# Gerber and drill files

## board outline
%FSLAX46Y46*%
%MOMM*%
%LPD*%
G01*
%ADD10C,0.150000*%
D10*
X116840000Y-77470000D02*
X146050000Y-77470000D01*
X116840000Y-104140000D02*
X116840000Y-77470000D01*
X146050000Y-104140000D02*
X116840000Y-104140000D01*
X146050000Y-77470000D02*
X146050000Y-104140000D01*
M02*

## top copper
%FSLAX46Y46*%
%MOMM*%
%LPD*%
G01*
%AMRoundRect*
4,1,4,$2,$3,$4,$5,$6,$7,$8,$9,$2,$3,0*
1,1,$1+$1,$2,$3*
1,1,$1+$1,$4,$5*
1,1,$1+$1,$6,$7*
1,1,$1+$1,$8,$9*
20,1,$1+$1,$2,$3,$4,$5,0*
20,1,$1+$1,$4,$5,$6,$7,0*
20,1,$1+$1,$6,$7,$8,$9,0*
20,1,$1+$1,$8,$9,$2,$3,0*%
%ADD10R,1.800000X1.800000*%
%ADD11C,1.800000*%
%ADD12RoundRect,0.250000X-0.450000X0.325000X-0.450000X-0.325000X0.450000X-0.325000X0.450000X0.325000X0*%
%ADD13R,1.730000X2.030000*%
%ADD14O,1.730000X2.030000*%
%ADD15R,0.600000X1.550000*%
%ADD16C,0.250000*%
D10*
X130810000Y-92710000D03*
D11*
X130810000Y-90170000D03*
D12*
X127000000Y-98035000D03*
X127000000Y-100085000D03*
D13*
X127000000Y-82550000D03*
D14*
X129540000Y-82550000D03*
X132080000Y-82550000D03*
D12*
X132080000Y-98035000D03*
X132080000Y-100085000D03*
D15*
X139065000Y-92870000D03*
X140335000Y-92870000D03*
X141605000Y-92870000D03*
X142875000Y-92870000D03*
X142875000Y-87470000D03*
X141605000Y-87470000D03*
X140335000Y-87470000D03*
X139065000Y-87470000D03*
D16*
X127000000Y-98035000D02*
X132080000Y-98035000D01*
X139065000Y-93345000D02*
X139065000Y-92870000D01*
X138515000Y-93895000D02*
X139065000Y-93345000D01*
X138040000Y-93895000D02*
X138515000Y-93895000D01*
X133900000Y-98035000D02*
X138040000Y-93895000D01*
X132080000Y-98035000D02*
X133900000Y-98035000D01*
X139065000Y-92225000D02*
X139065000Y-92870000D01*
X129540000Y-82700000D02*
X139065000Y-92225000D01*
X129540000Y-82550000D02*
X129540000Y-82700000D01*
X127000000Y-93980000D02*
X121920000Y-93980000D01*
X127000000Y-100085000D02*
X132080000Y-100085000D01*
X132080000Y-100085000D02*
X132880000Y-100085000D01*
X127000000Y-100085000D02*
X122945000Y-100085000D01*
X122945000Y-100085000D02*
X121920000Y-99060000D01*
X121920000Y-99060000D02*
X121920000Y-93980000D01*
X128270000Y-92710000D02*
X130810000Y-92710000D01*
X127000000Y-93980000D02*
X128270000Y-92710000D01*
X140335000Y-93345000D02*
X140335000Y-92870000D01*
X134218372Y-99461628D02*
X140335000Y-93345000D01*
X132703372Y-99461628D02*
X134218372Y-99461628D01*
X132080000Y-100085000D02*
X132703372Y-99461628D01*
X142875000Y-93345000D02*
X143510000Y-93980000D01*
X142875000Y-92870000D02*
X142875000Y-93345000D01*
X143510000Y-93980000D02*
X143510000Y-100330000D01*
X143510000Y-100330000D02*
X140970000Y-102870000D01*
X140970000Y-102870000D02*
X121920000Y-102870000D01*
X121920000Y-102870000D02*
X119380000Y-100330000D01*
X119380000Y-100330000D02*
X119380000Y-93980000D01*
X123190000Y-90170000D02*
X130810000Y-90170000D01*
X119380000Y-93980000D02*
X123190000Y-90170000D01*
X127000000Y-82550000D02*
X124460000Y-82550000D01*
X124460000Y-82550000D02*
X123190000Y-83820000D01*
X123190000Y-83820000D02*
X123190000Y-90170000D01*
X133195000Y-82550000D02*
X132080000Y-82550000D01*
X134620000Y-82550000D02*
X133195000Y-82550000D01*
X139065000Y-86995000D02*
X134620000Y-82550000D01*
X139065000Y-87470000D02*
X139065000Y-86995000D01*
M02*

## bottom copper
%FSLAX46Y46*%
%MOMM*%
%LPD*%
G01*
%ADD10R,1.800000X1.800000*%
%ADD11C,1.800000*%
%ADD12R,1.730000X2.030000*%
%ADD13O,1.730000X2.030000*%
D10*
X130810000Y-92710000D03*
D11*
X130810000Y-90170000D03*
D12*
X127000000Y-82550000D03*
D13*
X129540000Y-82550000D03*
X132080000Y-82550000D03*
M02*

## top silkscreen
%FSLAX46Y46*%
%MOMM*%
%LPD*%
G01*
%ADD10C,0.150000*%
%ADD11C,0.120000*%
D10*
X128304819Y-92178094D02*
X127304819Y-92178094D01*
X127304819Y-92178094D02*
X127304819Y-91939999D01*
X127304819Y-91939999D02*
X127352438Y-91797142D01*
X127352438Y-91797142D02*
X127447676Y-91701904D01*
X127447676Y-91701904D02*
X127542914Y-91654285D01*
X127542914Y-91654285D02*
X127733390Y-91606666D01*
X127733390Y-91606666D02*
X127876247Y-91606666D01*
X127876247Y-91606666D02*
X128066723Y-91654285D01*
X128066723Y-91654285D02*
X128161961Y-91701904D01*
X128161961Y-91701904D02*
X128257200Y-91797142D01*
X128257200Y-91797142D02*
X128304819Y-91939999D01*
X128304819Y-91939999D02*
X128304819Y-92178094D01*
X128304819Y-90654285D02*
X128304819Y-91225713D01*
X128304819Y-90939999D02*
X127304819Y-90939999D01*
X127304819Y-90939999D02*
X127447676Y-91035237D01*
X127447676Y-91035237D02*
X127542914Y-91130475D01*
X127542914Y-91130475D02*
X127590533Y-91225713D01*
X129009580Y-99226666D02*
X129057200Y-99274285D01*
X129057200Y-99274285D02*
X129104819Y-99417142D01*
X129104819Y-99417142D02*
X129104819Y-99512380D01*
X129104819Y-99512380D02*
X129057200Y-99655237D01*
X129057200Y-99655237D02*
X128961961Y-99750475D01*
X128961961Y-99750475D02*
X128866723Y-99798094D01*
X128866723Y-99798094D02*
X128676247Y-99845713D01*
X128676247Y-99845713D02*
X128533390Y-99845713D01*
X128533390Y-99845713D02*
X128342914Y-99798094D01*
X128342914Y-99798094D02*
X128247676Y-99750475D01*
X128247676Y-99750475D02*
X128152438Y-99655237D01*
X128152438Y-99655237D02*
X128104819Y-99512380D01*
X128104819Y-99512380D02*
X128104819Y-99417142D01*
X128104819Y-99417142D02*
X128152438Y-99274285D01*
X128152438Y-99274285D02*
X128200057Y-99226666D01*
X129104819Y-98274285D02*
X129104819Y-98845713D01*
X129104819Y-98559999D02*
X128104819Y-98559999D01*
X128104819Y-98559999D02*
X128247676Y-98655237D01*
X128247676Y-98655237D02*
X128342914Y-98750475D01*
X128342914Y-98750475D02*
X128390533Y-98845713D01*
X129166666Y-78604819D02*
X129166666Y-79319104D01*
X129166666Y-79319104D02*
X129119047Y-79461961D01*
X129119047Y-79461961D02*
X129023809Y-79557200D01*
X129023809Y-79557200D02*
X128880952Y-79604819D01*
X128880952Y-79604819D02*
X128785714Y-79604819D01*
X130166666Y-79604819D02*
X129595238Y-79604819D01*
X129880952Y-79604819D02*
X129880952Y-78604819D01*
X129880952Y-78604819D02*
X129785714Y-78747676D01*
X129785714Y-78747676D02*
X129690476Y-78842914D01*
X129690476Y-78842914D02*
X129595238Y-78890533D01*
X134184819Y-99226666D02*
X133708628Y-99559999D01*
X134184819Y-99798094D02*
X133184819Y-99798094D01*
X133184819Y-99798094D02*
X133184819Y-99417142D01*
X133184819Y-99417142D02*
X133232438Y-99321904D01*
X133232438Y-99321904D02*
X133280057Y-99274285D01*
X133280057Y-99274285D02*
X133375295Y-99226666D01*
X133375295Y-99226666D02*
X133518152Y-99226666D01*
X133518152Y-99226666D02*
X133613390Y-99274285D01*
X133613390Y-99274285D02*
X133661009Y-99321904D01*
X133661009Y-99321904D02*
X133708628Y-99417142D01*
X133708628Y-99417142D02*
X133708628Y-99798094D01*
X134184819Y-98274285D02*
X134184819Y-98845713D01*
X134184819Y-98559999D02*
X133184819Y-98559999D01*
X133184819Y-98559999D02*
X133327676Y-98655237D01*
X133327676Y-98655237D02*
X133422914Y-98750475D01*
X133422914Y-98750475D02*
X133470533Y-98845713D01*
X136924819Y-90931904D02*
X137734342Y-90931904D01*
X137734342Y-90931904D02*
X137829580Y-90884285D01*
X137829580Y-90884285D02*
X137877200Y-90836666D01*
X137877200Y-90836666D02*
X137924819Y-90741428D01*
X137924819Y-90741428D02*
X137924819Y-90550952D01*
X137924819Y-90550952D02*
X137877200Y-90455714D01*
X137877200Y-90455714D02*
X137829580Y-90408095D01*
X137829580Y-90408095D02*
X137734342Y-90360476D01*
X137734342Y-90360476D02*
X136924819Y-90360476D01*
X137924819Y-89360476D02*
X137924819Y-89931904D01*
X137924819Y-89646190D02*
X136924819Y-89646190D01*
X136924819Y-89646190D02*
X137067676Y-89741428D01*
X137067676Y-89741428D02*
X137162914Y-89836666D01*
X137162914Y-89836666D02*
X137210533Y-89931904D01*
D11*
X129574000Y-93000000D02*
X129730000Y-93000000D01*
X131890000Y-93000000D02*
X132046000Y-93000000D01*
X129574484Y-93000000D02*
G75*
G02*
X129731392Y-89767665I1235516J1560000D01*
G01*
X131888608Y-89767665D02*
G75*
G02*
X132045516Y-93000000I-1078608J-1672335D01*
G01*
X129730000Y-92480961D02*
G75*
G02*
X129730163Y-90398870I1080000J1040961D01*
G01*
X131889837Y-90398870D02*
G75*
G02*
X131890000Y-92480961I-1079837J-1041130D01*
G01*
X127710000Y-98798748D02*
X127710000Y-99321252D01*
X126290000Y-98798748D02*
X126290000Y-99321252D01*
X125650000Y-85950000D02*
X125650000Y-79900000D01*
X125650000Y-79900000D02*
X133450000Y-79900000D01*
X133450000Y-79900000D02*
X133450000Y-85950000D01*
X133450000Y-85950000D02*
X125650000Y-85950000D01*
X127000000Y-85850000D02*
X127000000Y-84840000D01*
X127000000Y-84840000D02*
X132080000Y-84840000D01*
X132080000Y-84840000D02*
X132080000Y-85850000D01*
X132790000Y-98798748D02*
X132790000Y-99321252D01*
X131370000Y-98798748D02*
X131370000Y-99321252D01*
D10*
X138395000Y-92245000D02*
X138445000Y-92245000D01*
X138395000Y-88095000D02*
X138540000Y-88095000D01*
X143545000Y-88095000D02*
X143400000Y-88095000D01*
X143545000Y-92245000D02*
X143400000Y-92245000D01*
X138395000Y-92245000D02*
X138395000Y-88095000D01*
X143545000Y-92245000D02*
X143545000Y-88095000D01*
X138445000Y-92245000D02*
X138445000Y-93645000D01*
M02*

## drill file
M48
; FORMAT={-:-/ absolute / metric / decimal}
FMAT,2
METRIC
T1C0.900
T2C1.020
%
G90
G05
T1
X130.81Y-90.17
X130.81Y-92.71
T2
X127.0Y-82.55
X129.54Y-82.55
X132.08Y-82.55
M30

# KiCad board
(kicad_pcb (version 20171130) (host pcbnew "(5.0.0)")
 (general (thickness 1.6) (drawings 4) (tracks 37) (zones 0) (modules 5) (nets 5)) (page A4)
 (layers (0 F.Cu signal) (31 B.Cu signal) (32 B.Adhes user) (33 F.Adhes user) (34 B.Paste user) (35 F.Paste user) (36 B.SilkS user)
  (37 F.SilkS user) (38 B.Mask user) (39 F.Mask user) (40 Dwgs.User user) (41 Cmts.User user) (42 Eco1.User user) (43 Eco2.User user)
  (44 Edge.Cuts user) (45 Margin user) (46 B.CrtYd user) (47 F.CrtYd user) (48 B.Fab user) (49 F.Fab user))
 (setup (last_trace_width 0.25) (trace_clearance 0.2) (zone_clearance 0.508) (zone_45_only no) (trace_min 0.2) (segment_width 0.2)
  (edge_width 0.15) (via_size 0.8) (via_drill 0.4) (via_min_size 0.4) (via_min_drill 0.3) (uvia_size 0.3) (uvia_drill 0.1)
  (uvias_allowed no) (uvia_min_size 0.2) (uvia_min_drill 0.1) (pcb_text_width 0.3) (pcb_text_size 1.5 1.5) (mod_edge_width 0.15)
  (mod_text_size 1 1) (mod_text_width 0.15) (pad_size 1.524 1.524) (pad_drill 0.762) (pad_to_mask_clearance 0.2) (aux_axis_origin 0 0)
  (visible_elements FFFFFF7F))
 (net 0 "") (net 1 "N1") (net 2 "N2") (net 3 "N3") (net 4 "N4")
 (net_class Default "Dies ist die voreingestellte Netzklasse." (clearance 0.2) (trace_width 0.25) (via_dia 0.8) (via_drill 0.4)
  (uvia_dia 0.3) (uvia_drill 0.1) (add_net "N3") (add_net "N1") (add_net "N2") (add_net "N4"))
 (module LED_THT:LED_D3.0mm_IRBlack (layer F.Cu) (at 130.81 92.71 90)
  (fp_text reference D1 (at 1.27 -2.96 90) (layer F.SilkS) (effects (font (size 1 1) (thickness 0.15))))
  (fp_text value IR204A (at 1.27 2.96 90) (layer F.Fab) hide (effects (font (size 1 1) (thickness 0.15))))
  (fp_line (start -0.29 -1.236) (end -0.29 -1.08) (layer F.SilkS) (width 0.12))
  (fp_line (start -0.29 1.08) (end -0.29 1.236) (layer F.SilkS) (width 0.12))
  (fp_arc (start 1.27 0) (end -0.29 -1.235516) (angle 108.8) (layer F.SilkS) (width 0.12))
  (fp_arc (start 1.27 0) (end -0.29 1.235516) (angle -108.8) (layer F.SilkS) (width 0.12))
  (fp_arc (start 1.27 0) (end 0.229039 -1.08) (angle 87.9) (layer F.SilkS) (width 0.12))
  (fp_arc (start 1.27 0) (end 0.229039 1.08) (angle -87.9) (layer F.SilkS) (width 0.12))
  (pad 1 thru_hole rect (at 0 0 90) (size 1.8 1.8) (drill 0.9) (layers *.Cu *.Mask) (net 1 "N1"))
  (pad 2 thru_hole circle (at 2.54 0 90) (size 1.8 1.8) (drill 0.9) (layers *.Cu *.Mask) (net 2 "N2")))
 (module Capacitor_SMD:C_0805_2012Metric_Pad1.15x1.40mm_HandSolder (layer F.Cu) (at 127 99.06 270)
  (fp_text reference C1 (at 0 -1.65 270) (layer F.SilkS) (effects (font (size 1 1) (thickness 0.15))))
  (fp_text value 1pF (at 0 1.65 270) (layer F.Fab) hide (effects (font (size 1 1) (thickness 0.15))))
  (fp_line (start -0.261252 -0.71) (end 0.261252 -0.71) (layer F.SilkS) (width 0.12))
  (fp_line (start -0.261252 0.71) (end 0.261252 0.71) (layer F.SilkS) (width 0.12))
  (pad 1 smd roundrect (at -1.025 0 270) (size 1.15 1.4) (layers F.Cu F.Paste F.Mask) (roundrect_rratio 0.217391) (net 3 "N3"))
  (pad 2 smd roundrect (at 1.025 0 270) (size 1.15 1.4) (layers F.Cu F.Paste F.Mask) (roundrect_rratio 0.217391) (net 1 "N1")))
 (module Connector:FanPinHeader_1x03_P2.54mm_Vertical (layer F.Cu) (at 127 82.55)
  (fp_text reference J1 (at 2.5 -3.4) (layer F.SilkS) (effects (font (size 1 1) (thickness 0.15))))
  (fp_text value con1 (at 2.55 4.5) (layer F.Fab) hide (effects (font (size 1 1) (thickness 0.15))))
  (fp_line (start -1.35 3.4) (end -1.35 -2.65) (layer F.SilkS) (width 0.12))
  (fp_line (start -1.35 -2.65) (end 6.45 -2.65) (layer F.SilkS) (width 0.12))
  (fp_line (start 6.45 -2.65) (end 6.45 3.4) (layer F.SilkS) (width 0.12))
  (fp_line (start 6.45 3.4) (end -1.35 3.4) (layer F.SilkS) (width 0.12))
  (fp_line (start 0 3.3) (end 0 2.29) (layer F.SilkS) (width 0.12))
  (fp_line (start 0 2.29) (end 5.08 2.29) (layer F.SilkS) (width 0.12))
  (fp_line (start 5.08 2.29) (end 5.08 3.3) (layer F.SilkS) (width 0.12))
  (pad 1 thru_hole rect (at 0 0 90) (size 2.03 1.73) (drill 1.02) (layers *.Cu *.Mask) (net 2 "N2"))
  (pad 2 thru_hole oval (at 2.54 0 90) (size 2.03 1.73) (drill 1.02) (layers *.Cu *.Mask) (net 3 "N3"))
  (pad 3 thru_hole oval (at 5.08 0 90) (size 2.03 1.73) (drill 1.02) (layers *.Cu *.Mask) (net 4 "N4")))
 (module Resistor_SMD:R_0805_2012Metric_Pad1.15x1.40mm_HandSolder (layer F.Cu) (at 132.08 99.06 270)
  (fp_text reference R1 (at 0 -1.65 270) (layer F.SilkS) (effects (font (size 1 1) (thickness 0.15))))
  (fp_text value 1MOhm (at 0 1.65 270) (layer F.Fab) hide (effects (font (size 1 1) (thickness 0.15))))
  (fp_line (start -0.261252 -0.71) (end 0.261252 -0.71) (layer F.SilkS) (width 0.12))
  (fp_line (start -0.261252 0.71) (end 0.261252 0.71) (layer F.SilkS) (width 0.12))
  (pad 1 smd roundrect (at -1.025 0 270) (size 1.15 1.4) (layers F.Cu F.Paste F.Mask) (roundrect_rratio 0.217391) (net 3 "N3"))
  (pad 2 smd roundrect (at 1.025 0 270) (size 1.15 1.4) (layers F.Cu F.Paste F.Mask) (roundrect_rratio 0.217391) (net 1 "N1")))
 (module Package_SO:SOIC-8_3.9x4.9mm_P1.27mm (layer F.Cu) (at 140.97 90.17 90)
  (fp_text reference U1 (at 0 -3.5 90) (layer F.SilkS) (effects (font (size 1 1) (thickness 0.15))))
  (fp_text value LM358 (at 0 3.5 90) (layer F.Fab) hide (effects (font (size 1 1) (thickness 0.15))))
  (fp_line (start -2.075 -2.575) (end -2.075 -2.525) (layer F.SilkS) (width 0.15))
  (fp_line (start 2.075 -2.575) (end 2.075 -2.43) (layer F.SilkS) (width 0.15))
  (fp_line (start 2.075 2.575) (end 2.075 2.43) (layer F.SilkS) (width 0.15))
  (fp_line (start -2.075 2.575) (end -2.075 2.43) (layer F.SilkS) (width 0.15))
  (fp_line (start -2.075 -2.575) (end 2.075 -2.575) (layer F.SilkS) (width 0.15))
  (fp_line (start -2.075 2.575) (end 2.075 2.575) (layer F.SilkS) (width 0.15))
  (fp_line (start -2.075 -2.525) (end -3.475 -2.525) (layer F.SilkS) (width 0.15))
  (pad 1 smd rect (at -2.7 -1.905 90) (size 1.55 0.6) (layers F.Cu F.Paste F.Mask) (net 3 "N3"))
  (pad 2 smd rect (at -2.7 -0.635 90) (size 1.55 0.6) (layers F.Cu F.Paste F.Mask) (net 1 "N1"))
  (pad 3 smd rect (at -2.7 0.635 90) (size 1.55 0.6) (layers F.Cu F.Paste F.Mask) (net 2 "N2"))
  (pad 4 smd rect (at -2.7 1.905 90) (size 1.55 0.6) (layers F.Cu F.Paste F.Mask) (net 2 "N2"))
  (pad 5 smd rect (at 2.7 1.905 90) (size 1.55 0.6) (layers F.Cu F.Paste F.Mask))
  (pad 6 smd rect (at 2.7 0.635 90) (size 1.55 0.6) (layers F.Cu F.Paste F.Mask))
  (pad 7 smd rect (at 2.7 -0.635 90) (size 1.55 0.6) (layers F.Cu F.Paste F.Mask))
  (pad 8 smd rect (at 2.7 -1.905 90) (size 1.55 0.6) (layers F.Cu F.Paste F.Mask) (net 4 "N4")))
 (gr_line (start 116.84 77.47) (end 146.05 77.47) (layer Edge.Cuts) (width 0.15))
 (gr_line (start 116.84 104.14) (end 116.84 77.47) (layer Edge.Cuts) (width 0.15))
 (gr_line (start 146.05 104.14) (end 116.84 104.14) (layer Edge.Cuts) (width 0.15))
 (gr_line (start 146.05 77.47) (end 146.05 104.14) (layer Edge.Cuts) (width 0.15))
 (segment (start 127 98.035) (end 132.08 98.035) (width 0.25) (layer F.Cu) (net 3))
 (segment (start 139.065 93.345) (end 139.065 92.87) (width 0.25) (layer F.Cu) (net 3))
 (segment (start 138.515 93.895) (end 139.065 93.345) (width 0.25) (layer F.Cu) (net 3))
 (segment (start 138.04 93.895) (end 138.515 93.895) (width 0.25) (layer F.Cu) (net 3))
 (segment (start 133.9 98.035) (end 138.04 93.895) (width 0.25) (layer F.Cu) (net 3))
 (segment (start 132.08 98.035) (end 133.9 98.035) (width 0.25) (layer F.Cu) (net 3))
 (segment (start 139.065 92.225) (end 139.065 92.87) (width 0.25) (layer F.Cu) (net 3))
 (segment (start 129.54 82.7) (end 139.065 92.225) (width 0.25) (layer F.Cu) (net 3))
 (segment (start 129.54 82.55) (end 129.54 82.7) (width 0.25) (layer F.Cu) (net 3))
 (segment (start 127 93.98) (end 121.92 93.98) (width 0.25) (layer F.Cu) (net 1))
 (segment (start 127 100.085) (end 132.08 100.085) (width 0.25) (layer F.Cu) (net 1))
 (segment (start 132.08 100.085) (end 132.88 100.085) (width 0.25) (layer F.Cu) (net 1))
 (segment (start 127 100.085) (end 122.945 100.085) (width 0.25) (layer F.Cu) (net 1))
 (segment (start 122.945 100.085) (end 121.92 99.06) (width 0.25) (layer F.Cu) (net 1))
 (segment (start 121.92 99.06) (end 121.92 93.98) (width 0.25) (layer F.Cu) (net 1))
 (segment (start 128.27 92.71) (end 130.81 92.71) (width 0.25) (layer F.Cu) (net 1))
 (segment (start 127 93.98) (end 128.27 92.71) (width 0.25) (layer F.Cu) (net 1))
 (segment (start 140.335 93.345) (end 140.335 92.87) (width 0.25) (layer F.Cu) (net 1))
 (segment (start 134.218372 99.461628) (end 140.335 93.345) (width 0.25) (layer F.Cu) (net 1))
 (segment (start 132.703372 99.461628) (end 134.218372 99.461628) (width 0.25) (layer F.Cu) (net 1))
 (segment (start 132.08 100.085) (end 132.703372 99.461628) (width 0.25) (layer F.Cu) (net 1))
 (segment (start 142.875 93.345) (end 143.51 93.98) (width 0.25) (layer F.Cu) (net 2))
 (segment (start 142.875 92.87) (end 142.875 93.345) (width 0.25) (layer F.Cu) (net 2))
 (segment (start 143.51 93.98) (end 143.51 100.33) (width 0.25) (layer F.Cu) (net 2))
 (segment (start 143.51 100.33) (end 140.97 102.87) (width 0.25) (layer F.Cu) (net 2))
 (segment (start 140.97 102.87) (end 121.92 102.87) (width 0.25) (layer F.Cu) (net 2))
 (segment (start 121.92 102.87) (end 119.38 100.33) (width 0.25) (layer F.Cu) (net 2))
 (segment (start 119.38 100.33) (end 119.38 93.98) (width 0.25) (layer F.Cu) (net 2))
 (segment (start 123.19 90.17) (end 130.81 90.17) (width 0.25) (layer F.Cu) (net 2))
 (segment (start 119.38 93.98) (end 123.19 90.17) (width 0.25) (layer F.Cu) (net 2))
 (segment (start 127 82.55) (end 124.46 82.55) (width 0.25) (layer F.Cu) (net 2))
 (segment (start 124.46 82.55) (end 123.19 83.82) (width 0.25) (layer F.Cu) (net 2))
 (segment (start 123.19 83.82) (end 123.19 90.17) (width 0.25) (layer F.Cu) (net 2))
 (segment (start 133.195 82.55) (end 132.08 82.55) (width 0.25) (layer F.Cu) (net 4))
 (segment (start 134.62 82.55) (end 133.195 82.55) (width 0.25) (layer F.Cu) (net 4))
 (segment (start 139.065 86.995) (end 134.62 82.55) (width 0.25) (layer F.Cu) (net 4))
 (segment (start 139.065 87.47) (end 139.065 86.995) (width 0.25) (layer F.Cu) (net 4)))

